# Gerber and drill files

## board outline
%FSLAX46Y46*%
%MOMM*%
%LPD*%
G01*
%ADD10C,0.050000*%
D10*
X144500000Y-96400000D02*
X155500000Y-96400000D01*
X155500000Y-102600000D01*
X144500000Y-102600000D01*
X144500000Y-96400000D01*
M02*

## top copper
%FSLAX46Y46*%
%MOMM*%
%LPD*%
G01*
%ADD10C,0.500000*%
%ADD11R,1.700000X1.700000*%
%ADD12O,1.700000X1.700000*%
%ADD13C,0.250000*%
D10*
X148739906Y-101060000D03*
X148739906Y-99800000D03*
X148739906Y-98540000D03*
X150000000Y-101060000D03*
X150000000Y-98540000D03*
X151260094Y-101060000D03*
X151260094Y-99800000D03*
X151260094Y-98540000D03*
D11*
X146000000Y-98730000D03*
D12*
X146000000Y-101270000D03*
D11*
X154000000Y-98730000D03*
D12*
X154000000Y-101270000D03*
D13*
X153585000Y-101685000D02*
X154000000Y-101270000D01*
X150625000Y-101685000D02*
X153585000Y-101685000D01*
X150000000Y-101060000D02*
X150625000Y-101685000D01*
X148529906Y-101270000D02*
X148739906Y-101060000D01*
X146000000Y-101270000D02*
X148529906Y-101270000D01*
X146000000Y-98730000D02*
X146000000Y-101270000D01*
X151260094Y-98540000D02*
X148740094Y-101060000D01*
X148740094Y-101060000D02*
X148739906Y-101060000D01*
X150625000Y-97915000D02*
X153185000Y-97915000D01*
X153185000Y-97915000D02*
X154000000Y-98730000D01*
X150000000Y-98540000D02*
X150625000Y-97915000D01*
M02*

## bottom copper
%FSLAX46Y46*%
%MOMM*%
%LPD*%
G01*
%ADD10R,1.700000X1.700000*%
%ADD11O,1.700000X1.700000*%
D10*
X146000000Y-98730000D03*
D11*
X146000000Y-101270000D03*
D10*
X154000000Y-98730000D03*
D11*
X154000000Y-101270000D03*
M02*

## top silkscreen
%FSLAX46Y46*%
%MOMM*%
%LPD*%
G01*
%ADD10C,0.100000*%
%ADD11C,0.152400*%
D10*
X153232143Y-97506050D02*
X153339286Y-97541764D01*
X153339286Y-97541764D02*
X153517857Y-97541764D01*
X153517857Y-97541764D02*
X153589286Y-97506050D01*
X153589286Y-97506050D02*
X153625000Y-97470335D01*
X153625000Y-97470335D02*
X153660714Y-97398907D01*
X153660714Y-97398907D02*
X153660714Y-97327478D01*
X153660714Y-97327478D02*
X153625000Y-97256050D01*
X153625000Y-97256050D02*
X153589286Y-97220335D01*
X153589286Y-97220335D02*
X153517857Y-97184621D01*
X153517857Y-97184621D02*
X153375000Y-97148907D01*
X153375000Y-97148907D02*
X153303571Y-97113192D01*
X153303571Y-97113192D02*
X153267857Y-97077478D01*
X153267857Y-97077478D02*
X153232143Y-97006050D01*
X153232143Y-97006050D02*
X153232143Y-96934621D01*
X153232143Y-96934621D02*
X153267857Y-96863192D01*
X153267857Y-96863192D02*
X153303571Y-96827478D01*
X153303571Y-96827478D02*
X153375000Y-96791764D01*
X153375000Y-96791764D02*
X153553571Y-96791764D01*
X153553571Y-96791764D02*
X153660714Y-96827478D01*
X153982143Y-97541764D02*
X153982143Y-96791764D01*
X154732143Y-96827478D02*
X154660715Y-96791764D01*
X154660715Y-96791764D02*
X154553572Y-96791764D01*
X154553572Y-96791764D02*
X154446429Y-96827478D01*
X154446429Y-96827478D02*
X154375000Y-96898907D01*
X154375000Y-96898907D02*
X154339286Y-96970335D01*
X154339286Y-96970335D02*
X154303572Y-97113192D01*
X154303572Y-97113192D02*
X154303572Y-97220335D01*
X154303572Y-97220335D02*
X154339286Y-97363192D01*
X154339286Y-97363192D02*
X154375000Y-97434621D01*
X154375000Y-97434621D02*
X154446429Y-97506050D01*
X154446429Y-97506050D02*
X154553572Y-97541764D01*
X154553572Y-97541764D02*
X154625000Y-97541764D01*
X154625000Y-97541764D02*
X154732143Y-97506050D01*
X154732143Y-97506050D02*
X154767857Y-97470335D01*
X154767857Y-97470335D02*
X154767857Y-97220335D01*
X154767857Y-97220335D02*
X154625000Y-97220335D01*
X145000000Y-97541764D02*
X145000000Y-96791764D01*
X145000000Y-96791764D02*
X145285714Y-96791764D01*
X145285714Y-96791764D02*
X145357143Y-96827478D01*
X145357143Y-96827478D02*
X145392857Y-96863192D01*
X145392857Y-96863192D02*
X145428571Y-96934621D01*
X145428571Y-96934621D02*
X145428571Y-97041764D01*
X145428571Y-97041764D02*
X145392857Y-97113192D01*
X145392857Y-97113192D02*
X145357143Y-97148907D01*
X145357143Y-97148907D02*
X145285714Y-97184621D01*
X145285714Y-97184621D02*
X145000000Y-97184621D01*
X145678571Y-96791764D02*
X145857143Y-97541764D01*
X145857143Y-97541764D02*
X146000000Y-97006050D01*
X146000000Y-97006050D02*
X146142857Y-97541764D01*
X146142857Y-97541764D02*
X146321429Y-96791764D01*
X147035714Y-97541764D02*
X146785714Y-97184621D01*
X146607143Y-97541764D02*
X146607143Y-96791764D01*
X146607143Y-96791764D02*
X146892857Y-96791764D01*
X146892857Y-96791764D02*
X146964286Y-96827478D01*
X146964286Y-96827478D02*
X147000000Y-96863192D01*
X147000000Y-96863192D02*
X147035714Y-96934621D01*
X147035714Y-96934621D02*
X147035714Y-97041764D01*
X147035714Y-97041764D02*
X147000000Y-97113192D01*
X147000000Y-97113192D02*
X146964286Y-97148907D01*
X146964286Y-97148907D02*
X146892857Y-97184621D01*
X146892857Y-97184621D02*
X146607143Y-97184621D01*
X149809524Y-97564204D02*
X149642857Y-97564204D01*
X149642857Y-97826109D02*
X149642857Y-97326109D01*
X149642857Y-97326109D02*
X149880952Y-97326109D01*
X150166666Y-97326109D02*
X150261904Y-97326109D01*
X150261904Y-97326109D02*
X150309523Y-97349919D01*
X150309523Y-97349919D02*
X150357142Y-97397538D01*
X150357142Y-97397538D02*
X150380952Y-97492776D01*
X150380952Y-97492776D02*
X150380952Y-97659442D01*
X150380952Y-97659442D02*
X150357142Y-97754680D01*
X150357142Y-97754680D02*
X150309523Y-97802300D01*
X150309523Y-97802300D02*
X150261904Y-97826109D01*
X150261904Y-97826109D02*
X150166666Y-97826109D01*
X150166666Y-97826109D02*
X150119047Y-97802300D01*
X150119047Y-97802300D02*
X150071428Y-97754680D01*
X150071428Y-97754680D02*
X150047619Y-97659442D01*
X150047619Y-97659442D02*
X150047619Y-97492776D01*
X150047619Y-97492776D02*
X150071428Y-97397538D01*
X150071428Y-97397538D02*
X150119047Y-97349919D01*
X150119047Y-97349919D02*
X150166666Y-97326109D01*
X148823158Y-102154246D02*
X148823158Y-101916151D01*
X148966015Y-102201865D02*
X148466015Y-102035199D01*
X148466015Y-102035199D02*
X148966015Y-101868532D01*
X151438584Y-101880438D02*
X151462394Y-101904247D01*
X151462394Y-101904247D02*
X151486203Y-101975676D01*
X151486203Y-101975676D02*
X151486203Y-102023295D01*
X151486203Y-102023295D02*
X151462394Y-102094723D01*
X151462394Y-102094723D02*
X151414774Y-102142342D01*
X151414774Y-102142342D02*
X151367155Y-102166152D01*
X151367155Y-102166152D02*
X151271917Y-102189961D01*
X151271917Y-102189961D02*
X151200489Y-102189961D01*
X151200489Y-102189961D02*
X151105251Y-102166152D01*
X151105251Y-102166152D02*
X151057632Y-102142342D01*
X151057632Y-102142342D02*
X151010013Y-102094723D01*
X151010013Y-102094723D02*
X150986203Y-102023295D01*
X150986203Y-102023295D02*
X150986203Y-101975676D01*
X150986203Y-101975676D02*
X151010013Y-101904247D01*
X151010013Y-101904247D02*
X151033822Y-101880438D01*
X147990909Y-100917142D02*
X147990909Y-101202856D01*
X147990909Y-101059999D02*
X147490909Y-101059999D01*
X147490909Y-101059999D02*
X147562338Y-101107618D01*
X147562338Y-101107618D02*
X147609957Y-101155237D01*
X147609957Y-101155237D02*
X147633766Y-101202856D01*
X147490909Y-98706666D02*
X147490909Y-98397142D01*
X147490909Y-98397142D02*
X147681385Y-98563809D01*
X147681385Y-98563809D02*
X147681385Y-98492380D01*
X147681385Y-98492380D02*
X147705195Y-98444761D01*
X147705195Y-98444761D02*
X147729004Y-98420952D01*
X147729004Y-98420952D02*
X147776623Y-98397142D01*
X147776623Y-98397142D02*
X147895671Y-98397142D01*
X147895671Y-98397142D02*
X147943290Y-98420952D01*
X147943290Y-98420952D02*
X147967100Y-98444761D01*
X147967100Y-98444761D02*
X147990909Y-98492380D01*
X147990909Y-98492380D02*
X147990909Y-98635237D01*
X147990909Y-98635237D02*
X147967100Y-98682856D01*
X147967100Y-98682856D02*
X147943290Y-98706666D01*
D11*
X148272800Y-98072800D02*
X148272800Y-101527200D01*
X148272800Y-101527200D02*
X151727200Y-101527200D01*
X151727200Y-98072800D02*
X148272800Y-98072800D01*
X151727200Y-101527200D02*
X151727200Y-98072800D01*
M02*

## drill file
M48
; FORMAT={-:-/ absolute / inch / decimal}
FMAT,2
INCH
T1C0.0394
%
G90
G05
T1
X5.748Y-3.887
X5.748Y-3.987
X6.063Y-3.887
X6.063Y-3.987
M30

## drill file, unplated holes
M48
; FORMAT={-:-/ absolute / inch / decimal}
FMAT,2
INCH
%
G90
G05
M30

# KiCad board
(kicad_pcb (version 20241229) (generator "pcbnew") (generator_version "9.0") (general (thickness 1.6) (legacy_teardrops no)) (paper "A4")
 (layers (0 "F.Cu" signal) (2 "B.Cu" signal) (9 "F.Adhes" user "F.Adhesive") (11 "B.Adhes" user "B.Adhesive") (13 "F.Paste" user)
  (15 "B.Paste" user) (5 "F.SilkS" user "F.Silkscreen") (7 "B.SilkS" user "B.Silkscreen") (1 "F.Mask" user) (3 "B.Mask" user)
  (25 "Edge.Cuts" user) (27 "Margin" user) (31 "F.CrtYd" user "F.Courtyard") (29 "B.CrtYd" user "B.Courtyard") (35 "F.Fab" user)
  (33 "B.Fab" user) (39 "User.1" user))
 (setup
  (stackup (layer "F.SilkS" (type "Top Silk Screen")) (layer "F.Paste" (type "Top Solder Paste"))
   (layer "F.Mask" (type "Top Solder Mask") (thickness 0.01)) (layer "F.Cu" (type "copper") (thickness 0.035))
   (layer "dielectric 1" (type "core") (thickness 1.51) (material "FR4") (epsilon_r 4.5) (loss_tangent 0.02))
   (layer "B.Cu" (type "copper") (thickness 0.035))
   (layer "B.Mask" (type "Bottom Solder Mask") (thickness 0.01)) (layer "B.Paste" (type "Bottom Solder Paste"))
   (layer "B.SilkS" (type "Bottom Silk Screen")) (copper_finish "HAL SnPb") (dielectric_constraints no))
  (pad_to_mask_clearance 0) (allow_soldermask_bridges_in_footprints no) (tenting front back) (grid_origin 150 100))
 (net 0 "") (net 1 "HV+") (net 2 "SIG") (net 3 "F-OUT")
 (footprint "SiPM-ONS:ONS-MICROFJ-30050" (layer "F.Cu") (at 150 99.8 90)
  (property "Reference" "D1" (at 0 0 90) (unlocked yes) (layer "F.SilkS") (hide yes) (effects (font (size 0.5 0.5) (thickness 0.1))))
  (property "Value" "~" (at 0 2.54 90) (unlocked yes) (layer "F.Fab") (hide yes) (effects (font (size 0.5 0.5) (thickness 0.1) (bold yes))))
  (fp_line (start 1.7272 -1.7272) (end -1.7272 -1.7272) (stroke (width 0.1524) (type solid)) (layer "F.SilkS"))
  (fp_line (start -1.7272 -1.7272) (end -1.7272 1.7272) (stroke (width 0.1524) (type solid)) (layer "F.SilkS"))
  (fp_line (start 1.7272 1.7272) (end 1.7272 -1.7272) (stroke (width 0.1524) (type solid)) (layer "F.SilkS"))
  (fp_line (start -1.7272 1.7272) (end 1.7272 1.7272) (stroke (width 0.1524) (type solid)) (layer "F.SilkS"))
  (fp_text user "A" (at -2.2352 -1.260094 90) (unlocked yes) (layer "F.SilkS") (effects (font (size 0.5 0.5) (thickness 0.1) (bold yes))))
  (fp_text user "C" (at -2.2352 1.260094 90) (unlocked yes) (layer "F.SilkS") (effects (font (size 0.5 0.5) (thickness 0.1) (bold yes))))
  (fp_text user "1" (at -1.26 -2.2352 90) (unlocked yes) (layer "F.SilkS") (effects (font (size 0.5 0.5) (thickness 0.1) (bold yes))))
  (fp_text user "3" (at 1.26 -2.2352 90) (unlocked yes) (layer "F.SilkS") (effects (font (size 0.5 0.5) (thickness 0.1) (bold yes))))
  (pad "A1" smd circle (at -1.26 -1.260094 90) (size 0.5 0.5) (layers "F.Cu" "F.Mask" "F.Paste") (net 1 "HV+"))
  (pad "A2" smd circle (at 0 -1.260094 90) (size 0.5 0.5) (layers "F.Cu" "F.Mask" "F.Paste"))
  (pad "A3" smd circle (at 1.26 -1.260094 90) (size 0.5 0.5) (layers "F.Cu" "F.Mask" "F.Paste"))
  (pad "B1" smd circle (at -1.26 0 90) (size 0.5 0.5) (layers "F.Cu" "F.Mask" "F.Paste") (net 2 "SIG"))
  (pad "B3" smd circle (at 1.26 0 90) (size 0.5 0.5) (layers "F.Cu" "F.Mask" "F.Paste") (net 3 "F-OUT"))
  (pad "C1" smd circle (at -1.26 1.260094 90) (size 0.5 0.5) (layers "F.Cu" "F.Mask" "F.Paste"))
  (pad "C2" smd circle (at 0 1.260094 90) (size 0.5 0.5) (layers "F.Cu" "F.Mask" "F.Paste"))
  (pad "C3" smd circle (at 1.26 1.260094 90) (size 0.5 0.5) (layers "F.Cu" "F.Mask" "F.Paste") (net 1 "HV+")))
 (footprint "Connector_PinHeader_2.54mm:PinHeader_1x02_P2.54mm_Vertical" (layer "F.Cu") (at 146 98.73)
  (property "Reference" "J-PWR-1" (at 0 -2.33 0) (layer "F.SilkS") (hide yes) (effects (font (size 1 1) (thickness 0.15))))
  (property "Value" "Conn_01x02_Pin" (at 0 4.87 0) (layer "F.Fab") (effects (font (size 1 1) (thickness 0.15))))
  (pad "1" thru_hole rect (at 0 0) (size 1.7 1.7) (drill 1) (layers "*.Cu" "*.Mask") (remove_unused_layers no) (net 1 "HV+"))
  (pad "2" thru_hole oval (at 0 2.54) (size 1.7 1.7) (drill 1) (layers "*.Cu" "*.Mask") (remove_unused_layers no) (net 1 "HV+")))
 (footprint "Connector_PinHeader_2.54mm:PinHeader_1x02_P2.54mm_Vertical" (layer "F.Cu") (at 154 98.73)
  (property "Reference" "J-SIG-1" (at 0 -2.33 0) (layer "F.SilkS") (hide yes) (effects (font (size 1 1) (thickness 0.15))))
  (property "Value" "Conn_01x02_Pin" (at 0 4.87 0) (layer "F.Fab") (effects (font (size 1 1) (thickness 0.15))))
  (pad "1" thru_hole rect (at 0 0) (size 1.7 1.7) (drill 1) (layers "*.Cu" "*.Mask") (remove_unused_layers no) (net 3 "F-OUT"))
  (pad "2" thru_hole oval (at 0 2.54) (size 1.7 1.7) (drill 1) (layers "*.Cu" "*.Mask") (remove_unused_layers no) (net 2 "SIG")))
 (gr_rect (start 144.5 96.4) (end 155.5 102.6) (stroke (width 0.05) (type default)) (fill no) (layer "Edge.Cuts"))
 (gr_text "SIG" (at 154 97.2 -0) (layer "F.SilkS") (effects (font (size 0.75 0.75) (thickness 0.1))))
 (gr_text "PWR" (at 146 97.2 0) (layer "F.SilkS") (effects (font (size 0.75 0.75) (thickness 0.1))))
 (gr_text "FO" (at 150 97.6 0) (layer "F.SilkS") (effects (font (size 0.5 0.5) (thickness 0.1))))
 (segment (start 153.585 101.685) (end 154 101.27) (width 0.25) (layer "F.Cu") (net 2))
 (segment (start 150.625 101.685) (end 153.585 101.685) (width 0.25) (layer "F.Cu") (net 2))
 (segment (start 150 101.06) (end 150.625 101.685) (width 0.25) (layer "F.Cu") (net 2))
 (segment (start 148.529906 101.27) (end 148.739906 101.06) (width 0.25) (layer "F.Cu") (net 1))
 (segment (start 146 101.27) (end 148.529906 101.27) (width 0.25) (layer "F.Cu") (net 1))
 (segment (start 146 98.73) (end 146 101.27) (width 0.25) (layer "F.Cu") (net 1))
 (segment (start 151.260094 98.54) (end 148.740094 101.06) (width 0.25) (layer "F.Cu") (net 1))
 (segment (start 148.740094 101.06) (end 148.739906 101.06) (width 0.25) (layer "F.Cu") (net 1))
 (segment (start 150.625 97.915) (end 153.185 97.915) (width 0.25) (layer "F.Cu") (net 3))
 (segment (start 153.185 97.915) (end 154 98.73) (width 0.25) (layer "F.Cu") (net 3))
 (segment (start 150 98.54) (end 150.625 97.915) (width 0.25) (layer "F.Cu") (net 3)))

